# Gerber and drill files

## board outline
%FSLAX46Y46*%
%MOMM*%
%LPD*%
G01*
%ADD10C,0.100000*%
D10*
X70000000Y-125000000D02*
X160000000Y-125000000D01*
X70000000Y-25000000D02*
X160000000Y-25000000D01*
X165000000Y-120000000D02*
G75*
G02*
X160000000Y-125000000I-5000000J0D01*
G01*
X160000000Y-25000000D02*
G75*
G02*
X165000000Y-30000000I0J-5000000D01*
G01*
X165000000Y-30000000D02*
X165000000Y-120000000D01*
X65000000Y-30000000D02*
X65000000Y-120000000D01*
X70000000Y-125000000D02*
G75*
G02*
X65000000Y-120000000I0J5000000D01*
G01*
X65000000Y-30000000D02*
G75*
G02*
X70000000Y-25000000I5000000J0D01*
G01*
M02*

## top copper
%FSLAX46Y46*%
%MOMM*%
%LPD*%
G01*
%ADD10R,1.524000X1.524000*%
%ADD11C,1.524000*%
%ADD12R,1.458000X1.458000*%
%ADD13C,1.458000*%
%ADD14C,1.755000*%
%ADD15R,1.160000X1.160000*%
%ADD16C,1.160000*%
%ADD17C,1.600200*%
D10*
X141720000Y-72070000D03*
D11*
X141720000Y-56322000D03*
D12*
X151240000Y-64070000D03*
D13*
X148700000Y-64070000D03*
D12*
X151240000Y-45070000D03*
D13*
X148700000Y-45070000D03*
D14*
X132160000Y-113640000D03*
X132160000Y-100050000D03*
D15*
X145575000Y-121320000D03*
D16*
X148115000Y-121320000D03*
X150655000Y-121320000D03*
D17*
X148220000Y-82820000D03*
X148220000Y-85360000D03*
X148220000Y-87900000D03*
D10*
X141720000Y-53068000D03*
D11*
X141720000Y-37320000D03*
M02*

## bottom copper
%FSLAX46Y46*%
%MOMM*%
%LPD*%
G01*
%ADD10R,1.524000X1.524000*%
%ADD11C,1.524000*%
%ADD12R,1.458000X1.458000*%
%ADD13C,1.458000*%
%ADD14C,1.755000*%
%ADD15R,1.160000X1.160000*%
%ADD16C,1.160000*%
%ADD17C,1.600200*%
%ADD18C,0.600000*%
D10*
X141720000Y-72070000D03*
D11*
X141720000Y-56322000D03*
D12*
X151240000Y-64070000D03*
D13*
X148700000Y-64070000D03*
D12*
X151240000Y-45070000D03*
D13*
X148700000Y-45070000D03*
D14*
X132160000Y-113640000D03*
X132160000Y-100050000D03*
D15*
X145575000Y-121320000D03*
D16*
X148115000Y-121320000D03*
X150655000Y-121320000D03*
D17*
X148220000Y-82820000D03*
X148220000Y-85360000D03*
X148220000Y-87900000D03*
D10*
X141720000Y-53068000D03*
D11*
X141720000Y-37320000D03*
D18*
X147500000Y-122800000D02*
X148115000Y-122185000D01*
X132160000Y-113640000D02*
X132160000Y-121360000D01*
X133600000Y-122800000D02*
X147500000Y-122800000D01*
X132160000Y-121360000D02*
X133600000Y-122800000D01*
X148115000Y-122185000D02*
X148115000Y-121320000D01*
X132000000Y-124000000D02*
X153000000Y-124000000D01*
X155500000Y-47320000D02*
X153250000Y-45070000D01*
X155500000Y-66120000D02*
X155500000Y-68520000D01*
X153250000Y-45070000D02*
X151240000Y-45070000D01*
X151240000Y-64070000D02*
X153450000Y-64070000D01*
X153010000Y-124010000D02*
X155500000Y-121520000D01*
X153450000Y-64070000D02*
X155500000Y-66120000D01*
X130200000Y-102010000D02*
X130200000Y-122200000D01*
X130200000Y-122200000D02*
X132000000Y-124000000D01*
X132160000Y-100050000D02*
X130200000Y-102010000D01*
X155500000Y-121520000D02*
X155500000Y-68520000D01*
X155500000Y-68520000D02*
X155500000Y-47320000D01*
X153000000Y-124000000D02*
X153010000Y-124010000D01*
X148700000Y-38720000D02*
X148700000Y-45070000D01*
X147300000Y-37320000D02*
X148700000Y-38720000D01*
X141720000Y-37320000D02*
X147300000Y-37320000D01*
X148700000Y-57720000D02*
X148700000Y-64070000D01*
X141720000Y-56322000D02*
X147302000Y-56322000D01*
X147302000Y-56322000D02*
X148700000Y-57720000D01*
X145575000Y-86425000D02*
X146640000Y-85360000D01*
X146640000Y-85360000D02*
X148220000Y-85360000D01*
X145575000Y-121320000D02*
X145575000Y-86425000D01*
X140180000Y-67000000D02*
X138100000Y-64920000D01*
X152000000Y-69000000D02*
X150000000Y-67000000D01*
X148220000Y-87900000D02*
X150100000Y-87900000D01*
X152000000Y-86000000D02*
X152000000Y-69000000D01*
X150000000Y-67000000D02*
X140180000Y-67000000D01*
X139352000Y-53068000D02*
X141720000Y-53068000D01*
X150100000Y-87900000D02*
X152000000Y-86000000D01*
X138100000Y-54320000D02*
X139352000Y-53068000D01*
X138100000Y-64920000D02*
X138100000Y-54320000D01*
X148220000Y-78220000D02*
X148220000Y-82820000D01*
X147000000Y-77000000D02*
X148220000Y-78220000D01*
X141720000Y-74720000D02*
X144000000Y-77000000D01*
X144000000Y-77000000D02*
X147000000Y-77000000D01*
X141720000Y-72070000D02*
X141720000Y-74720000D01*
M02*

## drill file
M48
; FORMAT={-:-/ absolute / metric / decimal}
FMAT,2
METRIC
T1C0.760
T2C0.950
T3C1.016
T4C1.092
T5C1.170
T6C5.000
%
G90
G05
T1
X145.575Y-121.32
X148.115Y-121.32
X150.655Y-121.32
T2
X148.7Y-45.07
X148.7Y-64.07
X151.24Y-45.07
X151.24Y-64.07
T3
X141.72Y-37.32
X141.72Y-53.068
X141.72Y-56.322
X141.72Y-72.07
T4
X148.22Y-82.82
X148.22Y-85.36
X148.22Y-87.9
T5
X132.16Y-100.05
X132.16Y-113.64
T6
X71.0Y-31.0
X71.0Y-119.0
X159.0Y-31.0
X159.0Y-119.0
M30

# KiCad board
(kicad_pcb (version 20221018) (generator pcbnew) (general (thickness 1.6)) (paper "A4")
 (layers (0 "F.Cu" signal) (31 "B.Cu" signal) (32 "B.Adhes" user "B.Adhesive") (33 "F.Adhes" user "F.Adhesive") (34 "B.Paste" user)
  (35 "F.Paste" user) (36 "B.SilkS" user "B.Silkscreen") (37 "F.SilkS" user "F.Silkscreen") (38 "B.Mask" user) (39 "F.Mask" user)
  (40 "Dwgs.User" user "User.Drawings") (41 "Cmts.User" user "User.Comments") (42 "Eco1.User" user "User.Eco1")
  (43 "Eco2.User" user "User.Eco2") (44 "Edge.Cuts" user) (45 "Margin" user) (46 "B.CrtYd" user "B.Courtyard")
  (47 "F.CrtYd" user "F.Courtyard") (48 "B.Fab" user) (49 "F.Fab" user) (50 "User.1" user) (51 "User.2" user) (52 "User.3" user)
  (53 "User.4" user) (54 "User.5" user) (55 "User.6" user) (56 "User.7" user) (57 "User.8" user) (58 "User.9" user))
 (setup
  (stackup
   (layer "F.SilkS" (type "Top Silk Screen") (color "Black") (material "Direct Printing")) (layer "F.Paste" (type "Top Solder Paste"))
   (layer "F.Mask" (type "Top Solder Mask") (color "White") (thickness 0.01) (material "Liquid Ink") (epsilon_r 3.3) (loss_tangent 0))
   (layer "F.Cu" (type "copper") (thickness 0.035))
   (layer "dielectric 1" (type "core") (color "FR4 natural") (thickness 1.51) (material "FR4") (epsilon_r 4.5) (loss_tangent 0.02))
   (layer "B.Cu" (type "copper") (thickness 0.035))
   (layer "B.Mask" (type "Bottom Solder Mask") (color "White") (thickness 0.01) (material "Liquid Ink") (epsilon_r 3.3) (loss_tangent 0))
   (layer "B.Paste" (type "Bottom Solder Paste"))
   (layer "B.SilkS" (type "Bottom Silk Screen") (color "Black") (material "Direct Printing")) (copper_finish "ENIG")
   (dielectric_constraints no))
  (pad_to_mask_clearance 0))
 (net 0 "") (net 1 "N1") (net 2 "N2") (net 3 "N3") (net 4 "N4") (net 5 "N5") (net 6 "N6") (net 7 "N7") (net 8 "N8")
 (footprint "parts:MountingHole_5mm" (layer "F.Cu") (at 71 31)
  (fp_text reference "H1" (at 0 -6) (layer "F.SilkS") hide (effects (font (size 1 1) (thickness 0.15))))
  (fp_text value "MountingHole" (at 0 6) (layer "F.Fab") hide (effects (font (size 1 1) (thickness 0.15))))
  (pad "" np_thru_hole circle (at 0 0) (size 5 5) (drill 5) (layers "*.Cu" "*.Mask")))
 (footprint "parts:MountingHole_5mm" (layer "F.Cu") (at 71 119)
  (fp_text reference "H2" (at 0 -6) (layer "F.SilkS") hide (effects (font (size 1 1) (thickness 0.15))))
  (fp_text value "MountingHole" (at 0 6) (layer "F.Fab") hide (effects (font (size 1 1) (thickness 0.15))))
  (pad "" np_thru_hole circle (at 0 0) (size 5 5) (drill 5) (layers "*.Cu" "*.Mask")))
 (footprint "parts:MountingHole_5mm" (layer "F.Cu") (at 159 31)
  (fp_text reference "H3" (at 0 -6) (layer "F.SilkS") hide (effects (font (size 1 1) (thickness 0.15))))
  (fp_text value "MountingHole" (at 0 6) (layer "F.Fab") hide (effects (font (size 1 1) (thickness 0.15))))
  (pad "" np_thru_hole circle (at 0 0) (size 5 5) (drill 5) (layers "*.Cu" "*.Mask")))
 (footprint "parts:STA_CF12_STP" (layer "F.Cu") (at 141.72 72.07 90)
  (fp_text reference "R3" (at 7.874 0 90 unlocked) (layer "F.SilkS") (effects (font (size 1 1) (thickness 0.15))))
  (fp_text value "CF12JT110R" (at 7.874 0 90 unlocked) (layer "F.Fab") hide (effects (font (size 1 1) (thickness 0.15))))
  (pad "1" thru_hole rect (at 0 0 90) (size 1.524 1.524) (drill 1.016) (layers "*.Cu" "*.Mask") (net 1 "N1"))
  (pad "2" thru_hole circle (at 15.748 0 90) (size 1.524 1.524) (drill 1.016) (layers "*.Cu" "*.Mask") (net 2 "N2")))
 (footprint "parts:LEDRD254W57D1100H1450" (layer "F.Cu") (at 149.97 64.07 180)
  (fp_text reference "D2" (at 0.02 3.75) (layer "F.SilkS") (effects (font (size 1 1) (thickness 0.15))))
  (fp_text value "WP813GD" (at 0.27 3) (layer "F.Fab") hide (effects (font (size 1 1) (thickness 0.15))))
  (pad "1" thru_hole rect (at -1.27 0 180) (size 1.458 1.458) (drill 0.95) (layers "*.Cu" "*.Mask") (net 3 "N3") (solder_mask_margin 0.102))
  (pad "2" thru_hole circle (at 1.27 0 180) (size 1.458 1.458) (drill 0.95) (layers "*.Cu" "*.Mask") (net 2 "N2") (solder_mask_margin 0.102)))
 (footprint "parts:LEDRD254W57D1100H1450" (layer "F.Cu") (at 149.97 45.07 180)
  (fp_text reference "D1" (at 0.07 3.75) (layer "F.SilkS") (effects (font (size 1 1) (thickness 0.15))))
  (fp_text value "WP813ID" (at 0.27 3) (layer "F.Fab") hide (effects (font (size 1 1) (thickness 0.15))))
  (pad "1" thru_hole rect (at -1.27 0 180) (size 1.458 1.458) (drill 0.95) (layers "*.Cu" "*.Mask") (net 3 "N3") (solder_mask_margin 0.102))
  (pad "2" thru_hole circle (at 1.27 0 180) (size 1.458 1.458) (drill 0.95) (layers "*.Cu" "*.Mask") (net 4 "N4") (solder_mask_margin 0.102)))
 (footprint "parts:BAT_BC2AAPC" (layer "F.Cu") (at 106 107 180)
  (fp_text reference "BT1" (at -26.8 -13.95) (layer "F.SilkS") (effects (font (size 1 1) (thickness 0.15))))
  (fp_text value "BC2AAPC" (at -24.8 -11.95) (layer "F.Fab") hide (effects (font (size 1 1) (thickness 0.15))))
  (pad "+" thru_hole circle (at -26.16 -6.64 180) (size 1.755 1.755) (drill 1.17) (layers "*.Cu" "*.Mask") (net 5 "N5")
   (solder_mask_margin 0.102))
  (pad "-" thru_hole circle (at -26.16 6.95 180) (size 1.755 1.755) (drill 1.17) (layers "*.Cu" "*.Mask") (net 3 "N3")
   (solder_mask_margin 0.102)))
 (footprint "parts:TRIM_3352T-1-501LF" (layer "F.Cu") (at 148.115 118.45)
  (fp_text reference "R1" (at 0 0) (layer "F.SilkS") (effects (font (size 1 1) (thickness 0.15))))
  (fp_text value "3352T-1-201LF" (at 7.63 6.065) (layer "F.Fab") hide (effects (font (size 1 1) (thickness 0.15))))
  (pad "1" thru_hole rect (at -2.54 2.87) (size 1.16 1.16) (drill 0.76) (layers "*.Cu" "*.Mask") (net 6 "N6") (solder_mask_margin 0.102))
  (pad "2" thru_hole circle (at 0 2.87) (size 1.16 1.16) (drill 0.76) (layers "*.Cu" "*.Mask") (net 5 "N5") (solder_mask_margin 0.102))
  (pad "3" thru_hole circle (at 2.54 2.87) (size 1.16 1.16) (drill 0.76) (layers "*.Cu" "*.Mask") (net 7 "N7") (solder_mask_margin 0.102)))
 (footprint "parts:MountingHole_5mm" (layer "F.Cu") (at 159 119)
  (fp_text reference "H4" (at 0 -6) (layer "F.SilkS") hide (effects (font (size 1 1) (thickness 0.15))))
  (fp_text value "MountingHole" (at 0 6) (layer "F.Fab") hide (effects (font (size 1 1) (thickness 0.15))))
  (pad "" np_thru_hole circle (at 0 0) (size 5 5) (drill 5) (layers "*.Cu" "*.Mask")))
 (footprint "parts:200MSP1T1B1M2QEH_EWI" (layer "F.Cu") (at 148.22 82.82 -90)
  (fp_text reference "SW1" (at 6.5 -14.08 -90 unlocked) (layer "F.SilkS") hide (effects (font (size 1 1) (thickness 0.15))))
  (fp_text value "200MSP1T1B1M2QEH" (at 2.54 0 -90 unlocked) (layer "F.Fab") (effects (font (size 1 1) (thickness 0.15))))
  (pad "1" thru_hole circle (at 0 0 270) (size 1.6002 1.6002) (drill 1.0922) (layers "*.Cu" "*.Mask") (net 1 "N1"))
  (pad "2" thru_hole circle (at 2.54 0 270) (size 1.6002 1.6002) (drill 1.0922) (layers "*.Cu" "*.Mask") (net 6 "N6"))
  (pad "3" thru_hole circle (at 5.08 0 270) (size 1.6002 1.6002) (drill 1.0922) (layers "*.Cu" "*.Mask") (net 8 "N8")))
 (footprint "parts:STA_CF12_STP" (layer "F.Cu") (at 141.72 53.068 90)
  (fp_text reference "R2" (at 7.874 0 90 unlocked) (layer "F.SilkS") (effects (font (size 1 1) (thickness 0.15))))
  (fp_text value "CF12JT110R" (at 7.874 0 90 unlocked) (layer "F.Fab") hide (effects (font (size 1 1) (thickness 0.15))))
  (pad "1" thru_hole rect (at 0 0 90) (size 1.524 1.524) (drill 1.016) (layers "*.Cu" "*.Mask") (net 8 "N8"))
  (pad "2" thru_hole circle (at 15.748 0 90) (size 1.524 1.524) (drill 1.016) (layers "*.Cu" "*.Mask") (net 4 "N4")))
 (gr_line (start 70 125) (end 160 125) (stroke (width 0.1) (type default)) (layer "Edge.Cuts"))
 (gr_line (start 70 25) (end 160 25) (stroke (width 0.1) (type default)) (layer "Edge.Cuts"))
 (gr_arc (start 165 120) (mid 163.535534 123.535534) (end 160 125) (stroke (width 0.1) (type default)) (layer "Edge.Cuts"))
 (gr_arc (start 160 25) (mid 163.535534 26.464466) (end 165 30) (stroke (width 0.1) (type default)) (layer "Edge.Cuts"))
 (gr_line (start 165 30) (end 165 120) (stroke (width 0.1) (type default)) (layer "Edge.Cuts"))
 (gr_line (start 65 30) (end 65 120) (stroke (width 0.1) (type default)) (layer "Edge.Cuts"))
 (gr_arc (start 70 125) (mid 66.464466 123.535534) (end 65 120) (stroke (width 0.1) (type default)) (layer "Edge.Cuts"))
 (gr_arc (start 65 30) (mid 66.464466 26.464466) (end 70 25) (stroke (width 0.1) (type default)) (layer "Edge.Cuts"))
 (segment (start 147.5 122.8) (end 148.115 122.185) (width 0.6) (layer "B.Cu") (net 5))
 (segment (start 132.16 113.64) (end 132.16 121.36) (width 0.6) (layer "B.Cu") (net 5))
 (segment (start 133.6 122.8) (end 147.5 122.8) (width 0.6) (layer "B.Cu") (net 5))
 (segment (start 132.16 121.36) (end 133.6 122.8) (width 0.6) (layer "B.Cu") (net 5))
 (segment (start 148.115 122.185) (end 148.115 121.32) (width 0.6) (layer "B.Cu") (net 5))
 (segment (start 132 124) (end 153 124) (width 0.6) (layer "B.Cu") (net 3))
 (segment (start 155.5 47.32) (end 153.25 45.07) (width 0.6) (layer "B.Cu") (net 3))
 (segment (start 155.5 66.12) (end 155.5 68.52) (width 0.6) (layer "B.Cu") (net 3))
 (segment (start 153.25 45.07) (end 151.24 45.07) (width 0.6) (layer "B.Cu") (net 3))
 (segment (start 151.24 64.07) (end 153.45 64.07) (width 0.6) (layer "B.Cu") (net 3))
 (segment (start 153.01 124.01) (end 155.5 121.52) (width 0.6) (layer "B.Cu") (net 3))
 (segment (start 153.45 64.07) (end 155.5 66.12) (width 0.6) (layer "B.Cu") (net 3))
 (segment (start 130.2 102.01) (end 130.2 122.2) (width 0.6) (layer "B.Cu") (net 3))
 (segment (start 130.2 122.2) (end 132 124) (width 0.6) (layer "B.Cu") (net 3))
 (segment (start 132.16 100.05) (end 130.2 102.01) (width 0.6) (layer "B.Cu") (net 3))
 (segment (start 155.5 121.52) (end 155.5 68.52) (width 0.6) (layer "B.Cu") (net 3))
 (segment (start 155.5 68.52) (end 155.5 47.32) (width 0.6) (layer "B.Cu") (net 3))
 (segment (start 153 124) (end 153.01 124.01) (width 0.6) (layer "B.Cu") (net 3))
 (segment (start 148.7 38.72) (end 148.7 45.07) (width 0.6) (layer "B.Cu") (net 4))
 (segment (start 147.3 37.32) (end 148.7 38.72) (width 0.6) (layer "B.Cu") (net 4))
 (segment (start 141.72 37.32) (end 147.3 37.32) (width 0.6) (layer "B.Cu") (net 4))
 (segment (start 148.7 57.72) (end 148.7 64.07) (width 0.6) (layer "B.Cu") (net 2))
 (segment (start 141.72 56.322) (end 147.302 56.322) (width 0.6) (layer "B.Cu") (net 2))
 (segment (start 147.302 56.322) (end 148.7 57.72) (width 0.6) (layer "B.Cu") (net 2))
 (segment (start 145.575 86.425) (end 146.64 85.36) (width 0.6) (layer "B.Cu") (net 6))
 (segment (start 146.64 85.36) (end 148.22 85.36) (width 0.6) (layer "B.Cu") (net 6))
 (segment (start 145.575 121.32) (end 145.575 86.425) (width 0.6) (layer "B.Cu") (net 6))
 (segment (start 140.18 67) (end 138.1 64.92) (width 0.6) (layer "B.Cu") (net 8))
 (segment (start 152 69) (end 150 67) (width 0.6) (layer "B.Cu") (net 8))
 (segment (start 148.22 87.9) (end 150.1 87.9) (width 0.6) (layer "B.Cu") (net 8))
 (segment (start 152 86) (end 152 69) (width 0.6) (layer "B.Cu") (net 8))
 (segment (start 150 67) (end 140.18 67) (width 0.6) (layer "B.Cu") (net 8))
 (segment (start 139.352 53.068) (end 141.72 53.068) (width 0.6) (layer "B.Cu") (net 8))
 (segment (start 150.1 87.9) (end 152 86) (width 0.6) (layer "B.Cu") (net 8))
 (segment (start 138.1 54.32) (end 139.352 53.068) (width 0.6) (layer "B.Cu") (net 8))
 (segment (start 138.1 64.92) (end 138.1 54.32) (width 0.6) (layer "B.Cu") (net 8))
 (segment (start 148.22 78.22) (end 148.22 82.82) (width 0.6) (layer "B.Cu") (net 1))
 (segment (start 147 77) (end 148.22 78.22) (width 0.6) (layer "B.Cu") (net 1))
 (segment (start 141.72 74.72) (end 144 77) (width 0.6) (layer "B.Cu") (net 1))
 (segment (start 144 77) (end 147 77) (width 0.6) (layer "B.Cu") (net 1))
 (segment (start 141.72 72.07) (end 141.72 74.72) (width 0.6) (layer "B.Cu") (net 1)))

